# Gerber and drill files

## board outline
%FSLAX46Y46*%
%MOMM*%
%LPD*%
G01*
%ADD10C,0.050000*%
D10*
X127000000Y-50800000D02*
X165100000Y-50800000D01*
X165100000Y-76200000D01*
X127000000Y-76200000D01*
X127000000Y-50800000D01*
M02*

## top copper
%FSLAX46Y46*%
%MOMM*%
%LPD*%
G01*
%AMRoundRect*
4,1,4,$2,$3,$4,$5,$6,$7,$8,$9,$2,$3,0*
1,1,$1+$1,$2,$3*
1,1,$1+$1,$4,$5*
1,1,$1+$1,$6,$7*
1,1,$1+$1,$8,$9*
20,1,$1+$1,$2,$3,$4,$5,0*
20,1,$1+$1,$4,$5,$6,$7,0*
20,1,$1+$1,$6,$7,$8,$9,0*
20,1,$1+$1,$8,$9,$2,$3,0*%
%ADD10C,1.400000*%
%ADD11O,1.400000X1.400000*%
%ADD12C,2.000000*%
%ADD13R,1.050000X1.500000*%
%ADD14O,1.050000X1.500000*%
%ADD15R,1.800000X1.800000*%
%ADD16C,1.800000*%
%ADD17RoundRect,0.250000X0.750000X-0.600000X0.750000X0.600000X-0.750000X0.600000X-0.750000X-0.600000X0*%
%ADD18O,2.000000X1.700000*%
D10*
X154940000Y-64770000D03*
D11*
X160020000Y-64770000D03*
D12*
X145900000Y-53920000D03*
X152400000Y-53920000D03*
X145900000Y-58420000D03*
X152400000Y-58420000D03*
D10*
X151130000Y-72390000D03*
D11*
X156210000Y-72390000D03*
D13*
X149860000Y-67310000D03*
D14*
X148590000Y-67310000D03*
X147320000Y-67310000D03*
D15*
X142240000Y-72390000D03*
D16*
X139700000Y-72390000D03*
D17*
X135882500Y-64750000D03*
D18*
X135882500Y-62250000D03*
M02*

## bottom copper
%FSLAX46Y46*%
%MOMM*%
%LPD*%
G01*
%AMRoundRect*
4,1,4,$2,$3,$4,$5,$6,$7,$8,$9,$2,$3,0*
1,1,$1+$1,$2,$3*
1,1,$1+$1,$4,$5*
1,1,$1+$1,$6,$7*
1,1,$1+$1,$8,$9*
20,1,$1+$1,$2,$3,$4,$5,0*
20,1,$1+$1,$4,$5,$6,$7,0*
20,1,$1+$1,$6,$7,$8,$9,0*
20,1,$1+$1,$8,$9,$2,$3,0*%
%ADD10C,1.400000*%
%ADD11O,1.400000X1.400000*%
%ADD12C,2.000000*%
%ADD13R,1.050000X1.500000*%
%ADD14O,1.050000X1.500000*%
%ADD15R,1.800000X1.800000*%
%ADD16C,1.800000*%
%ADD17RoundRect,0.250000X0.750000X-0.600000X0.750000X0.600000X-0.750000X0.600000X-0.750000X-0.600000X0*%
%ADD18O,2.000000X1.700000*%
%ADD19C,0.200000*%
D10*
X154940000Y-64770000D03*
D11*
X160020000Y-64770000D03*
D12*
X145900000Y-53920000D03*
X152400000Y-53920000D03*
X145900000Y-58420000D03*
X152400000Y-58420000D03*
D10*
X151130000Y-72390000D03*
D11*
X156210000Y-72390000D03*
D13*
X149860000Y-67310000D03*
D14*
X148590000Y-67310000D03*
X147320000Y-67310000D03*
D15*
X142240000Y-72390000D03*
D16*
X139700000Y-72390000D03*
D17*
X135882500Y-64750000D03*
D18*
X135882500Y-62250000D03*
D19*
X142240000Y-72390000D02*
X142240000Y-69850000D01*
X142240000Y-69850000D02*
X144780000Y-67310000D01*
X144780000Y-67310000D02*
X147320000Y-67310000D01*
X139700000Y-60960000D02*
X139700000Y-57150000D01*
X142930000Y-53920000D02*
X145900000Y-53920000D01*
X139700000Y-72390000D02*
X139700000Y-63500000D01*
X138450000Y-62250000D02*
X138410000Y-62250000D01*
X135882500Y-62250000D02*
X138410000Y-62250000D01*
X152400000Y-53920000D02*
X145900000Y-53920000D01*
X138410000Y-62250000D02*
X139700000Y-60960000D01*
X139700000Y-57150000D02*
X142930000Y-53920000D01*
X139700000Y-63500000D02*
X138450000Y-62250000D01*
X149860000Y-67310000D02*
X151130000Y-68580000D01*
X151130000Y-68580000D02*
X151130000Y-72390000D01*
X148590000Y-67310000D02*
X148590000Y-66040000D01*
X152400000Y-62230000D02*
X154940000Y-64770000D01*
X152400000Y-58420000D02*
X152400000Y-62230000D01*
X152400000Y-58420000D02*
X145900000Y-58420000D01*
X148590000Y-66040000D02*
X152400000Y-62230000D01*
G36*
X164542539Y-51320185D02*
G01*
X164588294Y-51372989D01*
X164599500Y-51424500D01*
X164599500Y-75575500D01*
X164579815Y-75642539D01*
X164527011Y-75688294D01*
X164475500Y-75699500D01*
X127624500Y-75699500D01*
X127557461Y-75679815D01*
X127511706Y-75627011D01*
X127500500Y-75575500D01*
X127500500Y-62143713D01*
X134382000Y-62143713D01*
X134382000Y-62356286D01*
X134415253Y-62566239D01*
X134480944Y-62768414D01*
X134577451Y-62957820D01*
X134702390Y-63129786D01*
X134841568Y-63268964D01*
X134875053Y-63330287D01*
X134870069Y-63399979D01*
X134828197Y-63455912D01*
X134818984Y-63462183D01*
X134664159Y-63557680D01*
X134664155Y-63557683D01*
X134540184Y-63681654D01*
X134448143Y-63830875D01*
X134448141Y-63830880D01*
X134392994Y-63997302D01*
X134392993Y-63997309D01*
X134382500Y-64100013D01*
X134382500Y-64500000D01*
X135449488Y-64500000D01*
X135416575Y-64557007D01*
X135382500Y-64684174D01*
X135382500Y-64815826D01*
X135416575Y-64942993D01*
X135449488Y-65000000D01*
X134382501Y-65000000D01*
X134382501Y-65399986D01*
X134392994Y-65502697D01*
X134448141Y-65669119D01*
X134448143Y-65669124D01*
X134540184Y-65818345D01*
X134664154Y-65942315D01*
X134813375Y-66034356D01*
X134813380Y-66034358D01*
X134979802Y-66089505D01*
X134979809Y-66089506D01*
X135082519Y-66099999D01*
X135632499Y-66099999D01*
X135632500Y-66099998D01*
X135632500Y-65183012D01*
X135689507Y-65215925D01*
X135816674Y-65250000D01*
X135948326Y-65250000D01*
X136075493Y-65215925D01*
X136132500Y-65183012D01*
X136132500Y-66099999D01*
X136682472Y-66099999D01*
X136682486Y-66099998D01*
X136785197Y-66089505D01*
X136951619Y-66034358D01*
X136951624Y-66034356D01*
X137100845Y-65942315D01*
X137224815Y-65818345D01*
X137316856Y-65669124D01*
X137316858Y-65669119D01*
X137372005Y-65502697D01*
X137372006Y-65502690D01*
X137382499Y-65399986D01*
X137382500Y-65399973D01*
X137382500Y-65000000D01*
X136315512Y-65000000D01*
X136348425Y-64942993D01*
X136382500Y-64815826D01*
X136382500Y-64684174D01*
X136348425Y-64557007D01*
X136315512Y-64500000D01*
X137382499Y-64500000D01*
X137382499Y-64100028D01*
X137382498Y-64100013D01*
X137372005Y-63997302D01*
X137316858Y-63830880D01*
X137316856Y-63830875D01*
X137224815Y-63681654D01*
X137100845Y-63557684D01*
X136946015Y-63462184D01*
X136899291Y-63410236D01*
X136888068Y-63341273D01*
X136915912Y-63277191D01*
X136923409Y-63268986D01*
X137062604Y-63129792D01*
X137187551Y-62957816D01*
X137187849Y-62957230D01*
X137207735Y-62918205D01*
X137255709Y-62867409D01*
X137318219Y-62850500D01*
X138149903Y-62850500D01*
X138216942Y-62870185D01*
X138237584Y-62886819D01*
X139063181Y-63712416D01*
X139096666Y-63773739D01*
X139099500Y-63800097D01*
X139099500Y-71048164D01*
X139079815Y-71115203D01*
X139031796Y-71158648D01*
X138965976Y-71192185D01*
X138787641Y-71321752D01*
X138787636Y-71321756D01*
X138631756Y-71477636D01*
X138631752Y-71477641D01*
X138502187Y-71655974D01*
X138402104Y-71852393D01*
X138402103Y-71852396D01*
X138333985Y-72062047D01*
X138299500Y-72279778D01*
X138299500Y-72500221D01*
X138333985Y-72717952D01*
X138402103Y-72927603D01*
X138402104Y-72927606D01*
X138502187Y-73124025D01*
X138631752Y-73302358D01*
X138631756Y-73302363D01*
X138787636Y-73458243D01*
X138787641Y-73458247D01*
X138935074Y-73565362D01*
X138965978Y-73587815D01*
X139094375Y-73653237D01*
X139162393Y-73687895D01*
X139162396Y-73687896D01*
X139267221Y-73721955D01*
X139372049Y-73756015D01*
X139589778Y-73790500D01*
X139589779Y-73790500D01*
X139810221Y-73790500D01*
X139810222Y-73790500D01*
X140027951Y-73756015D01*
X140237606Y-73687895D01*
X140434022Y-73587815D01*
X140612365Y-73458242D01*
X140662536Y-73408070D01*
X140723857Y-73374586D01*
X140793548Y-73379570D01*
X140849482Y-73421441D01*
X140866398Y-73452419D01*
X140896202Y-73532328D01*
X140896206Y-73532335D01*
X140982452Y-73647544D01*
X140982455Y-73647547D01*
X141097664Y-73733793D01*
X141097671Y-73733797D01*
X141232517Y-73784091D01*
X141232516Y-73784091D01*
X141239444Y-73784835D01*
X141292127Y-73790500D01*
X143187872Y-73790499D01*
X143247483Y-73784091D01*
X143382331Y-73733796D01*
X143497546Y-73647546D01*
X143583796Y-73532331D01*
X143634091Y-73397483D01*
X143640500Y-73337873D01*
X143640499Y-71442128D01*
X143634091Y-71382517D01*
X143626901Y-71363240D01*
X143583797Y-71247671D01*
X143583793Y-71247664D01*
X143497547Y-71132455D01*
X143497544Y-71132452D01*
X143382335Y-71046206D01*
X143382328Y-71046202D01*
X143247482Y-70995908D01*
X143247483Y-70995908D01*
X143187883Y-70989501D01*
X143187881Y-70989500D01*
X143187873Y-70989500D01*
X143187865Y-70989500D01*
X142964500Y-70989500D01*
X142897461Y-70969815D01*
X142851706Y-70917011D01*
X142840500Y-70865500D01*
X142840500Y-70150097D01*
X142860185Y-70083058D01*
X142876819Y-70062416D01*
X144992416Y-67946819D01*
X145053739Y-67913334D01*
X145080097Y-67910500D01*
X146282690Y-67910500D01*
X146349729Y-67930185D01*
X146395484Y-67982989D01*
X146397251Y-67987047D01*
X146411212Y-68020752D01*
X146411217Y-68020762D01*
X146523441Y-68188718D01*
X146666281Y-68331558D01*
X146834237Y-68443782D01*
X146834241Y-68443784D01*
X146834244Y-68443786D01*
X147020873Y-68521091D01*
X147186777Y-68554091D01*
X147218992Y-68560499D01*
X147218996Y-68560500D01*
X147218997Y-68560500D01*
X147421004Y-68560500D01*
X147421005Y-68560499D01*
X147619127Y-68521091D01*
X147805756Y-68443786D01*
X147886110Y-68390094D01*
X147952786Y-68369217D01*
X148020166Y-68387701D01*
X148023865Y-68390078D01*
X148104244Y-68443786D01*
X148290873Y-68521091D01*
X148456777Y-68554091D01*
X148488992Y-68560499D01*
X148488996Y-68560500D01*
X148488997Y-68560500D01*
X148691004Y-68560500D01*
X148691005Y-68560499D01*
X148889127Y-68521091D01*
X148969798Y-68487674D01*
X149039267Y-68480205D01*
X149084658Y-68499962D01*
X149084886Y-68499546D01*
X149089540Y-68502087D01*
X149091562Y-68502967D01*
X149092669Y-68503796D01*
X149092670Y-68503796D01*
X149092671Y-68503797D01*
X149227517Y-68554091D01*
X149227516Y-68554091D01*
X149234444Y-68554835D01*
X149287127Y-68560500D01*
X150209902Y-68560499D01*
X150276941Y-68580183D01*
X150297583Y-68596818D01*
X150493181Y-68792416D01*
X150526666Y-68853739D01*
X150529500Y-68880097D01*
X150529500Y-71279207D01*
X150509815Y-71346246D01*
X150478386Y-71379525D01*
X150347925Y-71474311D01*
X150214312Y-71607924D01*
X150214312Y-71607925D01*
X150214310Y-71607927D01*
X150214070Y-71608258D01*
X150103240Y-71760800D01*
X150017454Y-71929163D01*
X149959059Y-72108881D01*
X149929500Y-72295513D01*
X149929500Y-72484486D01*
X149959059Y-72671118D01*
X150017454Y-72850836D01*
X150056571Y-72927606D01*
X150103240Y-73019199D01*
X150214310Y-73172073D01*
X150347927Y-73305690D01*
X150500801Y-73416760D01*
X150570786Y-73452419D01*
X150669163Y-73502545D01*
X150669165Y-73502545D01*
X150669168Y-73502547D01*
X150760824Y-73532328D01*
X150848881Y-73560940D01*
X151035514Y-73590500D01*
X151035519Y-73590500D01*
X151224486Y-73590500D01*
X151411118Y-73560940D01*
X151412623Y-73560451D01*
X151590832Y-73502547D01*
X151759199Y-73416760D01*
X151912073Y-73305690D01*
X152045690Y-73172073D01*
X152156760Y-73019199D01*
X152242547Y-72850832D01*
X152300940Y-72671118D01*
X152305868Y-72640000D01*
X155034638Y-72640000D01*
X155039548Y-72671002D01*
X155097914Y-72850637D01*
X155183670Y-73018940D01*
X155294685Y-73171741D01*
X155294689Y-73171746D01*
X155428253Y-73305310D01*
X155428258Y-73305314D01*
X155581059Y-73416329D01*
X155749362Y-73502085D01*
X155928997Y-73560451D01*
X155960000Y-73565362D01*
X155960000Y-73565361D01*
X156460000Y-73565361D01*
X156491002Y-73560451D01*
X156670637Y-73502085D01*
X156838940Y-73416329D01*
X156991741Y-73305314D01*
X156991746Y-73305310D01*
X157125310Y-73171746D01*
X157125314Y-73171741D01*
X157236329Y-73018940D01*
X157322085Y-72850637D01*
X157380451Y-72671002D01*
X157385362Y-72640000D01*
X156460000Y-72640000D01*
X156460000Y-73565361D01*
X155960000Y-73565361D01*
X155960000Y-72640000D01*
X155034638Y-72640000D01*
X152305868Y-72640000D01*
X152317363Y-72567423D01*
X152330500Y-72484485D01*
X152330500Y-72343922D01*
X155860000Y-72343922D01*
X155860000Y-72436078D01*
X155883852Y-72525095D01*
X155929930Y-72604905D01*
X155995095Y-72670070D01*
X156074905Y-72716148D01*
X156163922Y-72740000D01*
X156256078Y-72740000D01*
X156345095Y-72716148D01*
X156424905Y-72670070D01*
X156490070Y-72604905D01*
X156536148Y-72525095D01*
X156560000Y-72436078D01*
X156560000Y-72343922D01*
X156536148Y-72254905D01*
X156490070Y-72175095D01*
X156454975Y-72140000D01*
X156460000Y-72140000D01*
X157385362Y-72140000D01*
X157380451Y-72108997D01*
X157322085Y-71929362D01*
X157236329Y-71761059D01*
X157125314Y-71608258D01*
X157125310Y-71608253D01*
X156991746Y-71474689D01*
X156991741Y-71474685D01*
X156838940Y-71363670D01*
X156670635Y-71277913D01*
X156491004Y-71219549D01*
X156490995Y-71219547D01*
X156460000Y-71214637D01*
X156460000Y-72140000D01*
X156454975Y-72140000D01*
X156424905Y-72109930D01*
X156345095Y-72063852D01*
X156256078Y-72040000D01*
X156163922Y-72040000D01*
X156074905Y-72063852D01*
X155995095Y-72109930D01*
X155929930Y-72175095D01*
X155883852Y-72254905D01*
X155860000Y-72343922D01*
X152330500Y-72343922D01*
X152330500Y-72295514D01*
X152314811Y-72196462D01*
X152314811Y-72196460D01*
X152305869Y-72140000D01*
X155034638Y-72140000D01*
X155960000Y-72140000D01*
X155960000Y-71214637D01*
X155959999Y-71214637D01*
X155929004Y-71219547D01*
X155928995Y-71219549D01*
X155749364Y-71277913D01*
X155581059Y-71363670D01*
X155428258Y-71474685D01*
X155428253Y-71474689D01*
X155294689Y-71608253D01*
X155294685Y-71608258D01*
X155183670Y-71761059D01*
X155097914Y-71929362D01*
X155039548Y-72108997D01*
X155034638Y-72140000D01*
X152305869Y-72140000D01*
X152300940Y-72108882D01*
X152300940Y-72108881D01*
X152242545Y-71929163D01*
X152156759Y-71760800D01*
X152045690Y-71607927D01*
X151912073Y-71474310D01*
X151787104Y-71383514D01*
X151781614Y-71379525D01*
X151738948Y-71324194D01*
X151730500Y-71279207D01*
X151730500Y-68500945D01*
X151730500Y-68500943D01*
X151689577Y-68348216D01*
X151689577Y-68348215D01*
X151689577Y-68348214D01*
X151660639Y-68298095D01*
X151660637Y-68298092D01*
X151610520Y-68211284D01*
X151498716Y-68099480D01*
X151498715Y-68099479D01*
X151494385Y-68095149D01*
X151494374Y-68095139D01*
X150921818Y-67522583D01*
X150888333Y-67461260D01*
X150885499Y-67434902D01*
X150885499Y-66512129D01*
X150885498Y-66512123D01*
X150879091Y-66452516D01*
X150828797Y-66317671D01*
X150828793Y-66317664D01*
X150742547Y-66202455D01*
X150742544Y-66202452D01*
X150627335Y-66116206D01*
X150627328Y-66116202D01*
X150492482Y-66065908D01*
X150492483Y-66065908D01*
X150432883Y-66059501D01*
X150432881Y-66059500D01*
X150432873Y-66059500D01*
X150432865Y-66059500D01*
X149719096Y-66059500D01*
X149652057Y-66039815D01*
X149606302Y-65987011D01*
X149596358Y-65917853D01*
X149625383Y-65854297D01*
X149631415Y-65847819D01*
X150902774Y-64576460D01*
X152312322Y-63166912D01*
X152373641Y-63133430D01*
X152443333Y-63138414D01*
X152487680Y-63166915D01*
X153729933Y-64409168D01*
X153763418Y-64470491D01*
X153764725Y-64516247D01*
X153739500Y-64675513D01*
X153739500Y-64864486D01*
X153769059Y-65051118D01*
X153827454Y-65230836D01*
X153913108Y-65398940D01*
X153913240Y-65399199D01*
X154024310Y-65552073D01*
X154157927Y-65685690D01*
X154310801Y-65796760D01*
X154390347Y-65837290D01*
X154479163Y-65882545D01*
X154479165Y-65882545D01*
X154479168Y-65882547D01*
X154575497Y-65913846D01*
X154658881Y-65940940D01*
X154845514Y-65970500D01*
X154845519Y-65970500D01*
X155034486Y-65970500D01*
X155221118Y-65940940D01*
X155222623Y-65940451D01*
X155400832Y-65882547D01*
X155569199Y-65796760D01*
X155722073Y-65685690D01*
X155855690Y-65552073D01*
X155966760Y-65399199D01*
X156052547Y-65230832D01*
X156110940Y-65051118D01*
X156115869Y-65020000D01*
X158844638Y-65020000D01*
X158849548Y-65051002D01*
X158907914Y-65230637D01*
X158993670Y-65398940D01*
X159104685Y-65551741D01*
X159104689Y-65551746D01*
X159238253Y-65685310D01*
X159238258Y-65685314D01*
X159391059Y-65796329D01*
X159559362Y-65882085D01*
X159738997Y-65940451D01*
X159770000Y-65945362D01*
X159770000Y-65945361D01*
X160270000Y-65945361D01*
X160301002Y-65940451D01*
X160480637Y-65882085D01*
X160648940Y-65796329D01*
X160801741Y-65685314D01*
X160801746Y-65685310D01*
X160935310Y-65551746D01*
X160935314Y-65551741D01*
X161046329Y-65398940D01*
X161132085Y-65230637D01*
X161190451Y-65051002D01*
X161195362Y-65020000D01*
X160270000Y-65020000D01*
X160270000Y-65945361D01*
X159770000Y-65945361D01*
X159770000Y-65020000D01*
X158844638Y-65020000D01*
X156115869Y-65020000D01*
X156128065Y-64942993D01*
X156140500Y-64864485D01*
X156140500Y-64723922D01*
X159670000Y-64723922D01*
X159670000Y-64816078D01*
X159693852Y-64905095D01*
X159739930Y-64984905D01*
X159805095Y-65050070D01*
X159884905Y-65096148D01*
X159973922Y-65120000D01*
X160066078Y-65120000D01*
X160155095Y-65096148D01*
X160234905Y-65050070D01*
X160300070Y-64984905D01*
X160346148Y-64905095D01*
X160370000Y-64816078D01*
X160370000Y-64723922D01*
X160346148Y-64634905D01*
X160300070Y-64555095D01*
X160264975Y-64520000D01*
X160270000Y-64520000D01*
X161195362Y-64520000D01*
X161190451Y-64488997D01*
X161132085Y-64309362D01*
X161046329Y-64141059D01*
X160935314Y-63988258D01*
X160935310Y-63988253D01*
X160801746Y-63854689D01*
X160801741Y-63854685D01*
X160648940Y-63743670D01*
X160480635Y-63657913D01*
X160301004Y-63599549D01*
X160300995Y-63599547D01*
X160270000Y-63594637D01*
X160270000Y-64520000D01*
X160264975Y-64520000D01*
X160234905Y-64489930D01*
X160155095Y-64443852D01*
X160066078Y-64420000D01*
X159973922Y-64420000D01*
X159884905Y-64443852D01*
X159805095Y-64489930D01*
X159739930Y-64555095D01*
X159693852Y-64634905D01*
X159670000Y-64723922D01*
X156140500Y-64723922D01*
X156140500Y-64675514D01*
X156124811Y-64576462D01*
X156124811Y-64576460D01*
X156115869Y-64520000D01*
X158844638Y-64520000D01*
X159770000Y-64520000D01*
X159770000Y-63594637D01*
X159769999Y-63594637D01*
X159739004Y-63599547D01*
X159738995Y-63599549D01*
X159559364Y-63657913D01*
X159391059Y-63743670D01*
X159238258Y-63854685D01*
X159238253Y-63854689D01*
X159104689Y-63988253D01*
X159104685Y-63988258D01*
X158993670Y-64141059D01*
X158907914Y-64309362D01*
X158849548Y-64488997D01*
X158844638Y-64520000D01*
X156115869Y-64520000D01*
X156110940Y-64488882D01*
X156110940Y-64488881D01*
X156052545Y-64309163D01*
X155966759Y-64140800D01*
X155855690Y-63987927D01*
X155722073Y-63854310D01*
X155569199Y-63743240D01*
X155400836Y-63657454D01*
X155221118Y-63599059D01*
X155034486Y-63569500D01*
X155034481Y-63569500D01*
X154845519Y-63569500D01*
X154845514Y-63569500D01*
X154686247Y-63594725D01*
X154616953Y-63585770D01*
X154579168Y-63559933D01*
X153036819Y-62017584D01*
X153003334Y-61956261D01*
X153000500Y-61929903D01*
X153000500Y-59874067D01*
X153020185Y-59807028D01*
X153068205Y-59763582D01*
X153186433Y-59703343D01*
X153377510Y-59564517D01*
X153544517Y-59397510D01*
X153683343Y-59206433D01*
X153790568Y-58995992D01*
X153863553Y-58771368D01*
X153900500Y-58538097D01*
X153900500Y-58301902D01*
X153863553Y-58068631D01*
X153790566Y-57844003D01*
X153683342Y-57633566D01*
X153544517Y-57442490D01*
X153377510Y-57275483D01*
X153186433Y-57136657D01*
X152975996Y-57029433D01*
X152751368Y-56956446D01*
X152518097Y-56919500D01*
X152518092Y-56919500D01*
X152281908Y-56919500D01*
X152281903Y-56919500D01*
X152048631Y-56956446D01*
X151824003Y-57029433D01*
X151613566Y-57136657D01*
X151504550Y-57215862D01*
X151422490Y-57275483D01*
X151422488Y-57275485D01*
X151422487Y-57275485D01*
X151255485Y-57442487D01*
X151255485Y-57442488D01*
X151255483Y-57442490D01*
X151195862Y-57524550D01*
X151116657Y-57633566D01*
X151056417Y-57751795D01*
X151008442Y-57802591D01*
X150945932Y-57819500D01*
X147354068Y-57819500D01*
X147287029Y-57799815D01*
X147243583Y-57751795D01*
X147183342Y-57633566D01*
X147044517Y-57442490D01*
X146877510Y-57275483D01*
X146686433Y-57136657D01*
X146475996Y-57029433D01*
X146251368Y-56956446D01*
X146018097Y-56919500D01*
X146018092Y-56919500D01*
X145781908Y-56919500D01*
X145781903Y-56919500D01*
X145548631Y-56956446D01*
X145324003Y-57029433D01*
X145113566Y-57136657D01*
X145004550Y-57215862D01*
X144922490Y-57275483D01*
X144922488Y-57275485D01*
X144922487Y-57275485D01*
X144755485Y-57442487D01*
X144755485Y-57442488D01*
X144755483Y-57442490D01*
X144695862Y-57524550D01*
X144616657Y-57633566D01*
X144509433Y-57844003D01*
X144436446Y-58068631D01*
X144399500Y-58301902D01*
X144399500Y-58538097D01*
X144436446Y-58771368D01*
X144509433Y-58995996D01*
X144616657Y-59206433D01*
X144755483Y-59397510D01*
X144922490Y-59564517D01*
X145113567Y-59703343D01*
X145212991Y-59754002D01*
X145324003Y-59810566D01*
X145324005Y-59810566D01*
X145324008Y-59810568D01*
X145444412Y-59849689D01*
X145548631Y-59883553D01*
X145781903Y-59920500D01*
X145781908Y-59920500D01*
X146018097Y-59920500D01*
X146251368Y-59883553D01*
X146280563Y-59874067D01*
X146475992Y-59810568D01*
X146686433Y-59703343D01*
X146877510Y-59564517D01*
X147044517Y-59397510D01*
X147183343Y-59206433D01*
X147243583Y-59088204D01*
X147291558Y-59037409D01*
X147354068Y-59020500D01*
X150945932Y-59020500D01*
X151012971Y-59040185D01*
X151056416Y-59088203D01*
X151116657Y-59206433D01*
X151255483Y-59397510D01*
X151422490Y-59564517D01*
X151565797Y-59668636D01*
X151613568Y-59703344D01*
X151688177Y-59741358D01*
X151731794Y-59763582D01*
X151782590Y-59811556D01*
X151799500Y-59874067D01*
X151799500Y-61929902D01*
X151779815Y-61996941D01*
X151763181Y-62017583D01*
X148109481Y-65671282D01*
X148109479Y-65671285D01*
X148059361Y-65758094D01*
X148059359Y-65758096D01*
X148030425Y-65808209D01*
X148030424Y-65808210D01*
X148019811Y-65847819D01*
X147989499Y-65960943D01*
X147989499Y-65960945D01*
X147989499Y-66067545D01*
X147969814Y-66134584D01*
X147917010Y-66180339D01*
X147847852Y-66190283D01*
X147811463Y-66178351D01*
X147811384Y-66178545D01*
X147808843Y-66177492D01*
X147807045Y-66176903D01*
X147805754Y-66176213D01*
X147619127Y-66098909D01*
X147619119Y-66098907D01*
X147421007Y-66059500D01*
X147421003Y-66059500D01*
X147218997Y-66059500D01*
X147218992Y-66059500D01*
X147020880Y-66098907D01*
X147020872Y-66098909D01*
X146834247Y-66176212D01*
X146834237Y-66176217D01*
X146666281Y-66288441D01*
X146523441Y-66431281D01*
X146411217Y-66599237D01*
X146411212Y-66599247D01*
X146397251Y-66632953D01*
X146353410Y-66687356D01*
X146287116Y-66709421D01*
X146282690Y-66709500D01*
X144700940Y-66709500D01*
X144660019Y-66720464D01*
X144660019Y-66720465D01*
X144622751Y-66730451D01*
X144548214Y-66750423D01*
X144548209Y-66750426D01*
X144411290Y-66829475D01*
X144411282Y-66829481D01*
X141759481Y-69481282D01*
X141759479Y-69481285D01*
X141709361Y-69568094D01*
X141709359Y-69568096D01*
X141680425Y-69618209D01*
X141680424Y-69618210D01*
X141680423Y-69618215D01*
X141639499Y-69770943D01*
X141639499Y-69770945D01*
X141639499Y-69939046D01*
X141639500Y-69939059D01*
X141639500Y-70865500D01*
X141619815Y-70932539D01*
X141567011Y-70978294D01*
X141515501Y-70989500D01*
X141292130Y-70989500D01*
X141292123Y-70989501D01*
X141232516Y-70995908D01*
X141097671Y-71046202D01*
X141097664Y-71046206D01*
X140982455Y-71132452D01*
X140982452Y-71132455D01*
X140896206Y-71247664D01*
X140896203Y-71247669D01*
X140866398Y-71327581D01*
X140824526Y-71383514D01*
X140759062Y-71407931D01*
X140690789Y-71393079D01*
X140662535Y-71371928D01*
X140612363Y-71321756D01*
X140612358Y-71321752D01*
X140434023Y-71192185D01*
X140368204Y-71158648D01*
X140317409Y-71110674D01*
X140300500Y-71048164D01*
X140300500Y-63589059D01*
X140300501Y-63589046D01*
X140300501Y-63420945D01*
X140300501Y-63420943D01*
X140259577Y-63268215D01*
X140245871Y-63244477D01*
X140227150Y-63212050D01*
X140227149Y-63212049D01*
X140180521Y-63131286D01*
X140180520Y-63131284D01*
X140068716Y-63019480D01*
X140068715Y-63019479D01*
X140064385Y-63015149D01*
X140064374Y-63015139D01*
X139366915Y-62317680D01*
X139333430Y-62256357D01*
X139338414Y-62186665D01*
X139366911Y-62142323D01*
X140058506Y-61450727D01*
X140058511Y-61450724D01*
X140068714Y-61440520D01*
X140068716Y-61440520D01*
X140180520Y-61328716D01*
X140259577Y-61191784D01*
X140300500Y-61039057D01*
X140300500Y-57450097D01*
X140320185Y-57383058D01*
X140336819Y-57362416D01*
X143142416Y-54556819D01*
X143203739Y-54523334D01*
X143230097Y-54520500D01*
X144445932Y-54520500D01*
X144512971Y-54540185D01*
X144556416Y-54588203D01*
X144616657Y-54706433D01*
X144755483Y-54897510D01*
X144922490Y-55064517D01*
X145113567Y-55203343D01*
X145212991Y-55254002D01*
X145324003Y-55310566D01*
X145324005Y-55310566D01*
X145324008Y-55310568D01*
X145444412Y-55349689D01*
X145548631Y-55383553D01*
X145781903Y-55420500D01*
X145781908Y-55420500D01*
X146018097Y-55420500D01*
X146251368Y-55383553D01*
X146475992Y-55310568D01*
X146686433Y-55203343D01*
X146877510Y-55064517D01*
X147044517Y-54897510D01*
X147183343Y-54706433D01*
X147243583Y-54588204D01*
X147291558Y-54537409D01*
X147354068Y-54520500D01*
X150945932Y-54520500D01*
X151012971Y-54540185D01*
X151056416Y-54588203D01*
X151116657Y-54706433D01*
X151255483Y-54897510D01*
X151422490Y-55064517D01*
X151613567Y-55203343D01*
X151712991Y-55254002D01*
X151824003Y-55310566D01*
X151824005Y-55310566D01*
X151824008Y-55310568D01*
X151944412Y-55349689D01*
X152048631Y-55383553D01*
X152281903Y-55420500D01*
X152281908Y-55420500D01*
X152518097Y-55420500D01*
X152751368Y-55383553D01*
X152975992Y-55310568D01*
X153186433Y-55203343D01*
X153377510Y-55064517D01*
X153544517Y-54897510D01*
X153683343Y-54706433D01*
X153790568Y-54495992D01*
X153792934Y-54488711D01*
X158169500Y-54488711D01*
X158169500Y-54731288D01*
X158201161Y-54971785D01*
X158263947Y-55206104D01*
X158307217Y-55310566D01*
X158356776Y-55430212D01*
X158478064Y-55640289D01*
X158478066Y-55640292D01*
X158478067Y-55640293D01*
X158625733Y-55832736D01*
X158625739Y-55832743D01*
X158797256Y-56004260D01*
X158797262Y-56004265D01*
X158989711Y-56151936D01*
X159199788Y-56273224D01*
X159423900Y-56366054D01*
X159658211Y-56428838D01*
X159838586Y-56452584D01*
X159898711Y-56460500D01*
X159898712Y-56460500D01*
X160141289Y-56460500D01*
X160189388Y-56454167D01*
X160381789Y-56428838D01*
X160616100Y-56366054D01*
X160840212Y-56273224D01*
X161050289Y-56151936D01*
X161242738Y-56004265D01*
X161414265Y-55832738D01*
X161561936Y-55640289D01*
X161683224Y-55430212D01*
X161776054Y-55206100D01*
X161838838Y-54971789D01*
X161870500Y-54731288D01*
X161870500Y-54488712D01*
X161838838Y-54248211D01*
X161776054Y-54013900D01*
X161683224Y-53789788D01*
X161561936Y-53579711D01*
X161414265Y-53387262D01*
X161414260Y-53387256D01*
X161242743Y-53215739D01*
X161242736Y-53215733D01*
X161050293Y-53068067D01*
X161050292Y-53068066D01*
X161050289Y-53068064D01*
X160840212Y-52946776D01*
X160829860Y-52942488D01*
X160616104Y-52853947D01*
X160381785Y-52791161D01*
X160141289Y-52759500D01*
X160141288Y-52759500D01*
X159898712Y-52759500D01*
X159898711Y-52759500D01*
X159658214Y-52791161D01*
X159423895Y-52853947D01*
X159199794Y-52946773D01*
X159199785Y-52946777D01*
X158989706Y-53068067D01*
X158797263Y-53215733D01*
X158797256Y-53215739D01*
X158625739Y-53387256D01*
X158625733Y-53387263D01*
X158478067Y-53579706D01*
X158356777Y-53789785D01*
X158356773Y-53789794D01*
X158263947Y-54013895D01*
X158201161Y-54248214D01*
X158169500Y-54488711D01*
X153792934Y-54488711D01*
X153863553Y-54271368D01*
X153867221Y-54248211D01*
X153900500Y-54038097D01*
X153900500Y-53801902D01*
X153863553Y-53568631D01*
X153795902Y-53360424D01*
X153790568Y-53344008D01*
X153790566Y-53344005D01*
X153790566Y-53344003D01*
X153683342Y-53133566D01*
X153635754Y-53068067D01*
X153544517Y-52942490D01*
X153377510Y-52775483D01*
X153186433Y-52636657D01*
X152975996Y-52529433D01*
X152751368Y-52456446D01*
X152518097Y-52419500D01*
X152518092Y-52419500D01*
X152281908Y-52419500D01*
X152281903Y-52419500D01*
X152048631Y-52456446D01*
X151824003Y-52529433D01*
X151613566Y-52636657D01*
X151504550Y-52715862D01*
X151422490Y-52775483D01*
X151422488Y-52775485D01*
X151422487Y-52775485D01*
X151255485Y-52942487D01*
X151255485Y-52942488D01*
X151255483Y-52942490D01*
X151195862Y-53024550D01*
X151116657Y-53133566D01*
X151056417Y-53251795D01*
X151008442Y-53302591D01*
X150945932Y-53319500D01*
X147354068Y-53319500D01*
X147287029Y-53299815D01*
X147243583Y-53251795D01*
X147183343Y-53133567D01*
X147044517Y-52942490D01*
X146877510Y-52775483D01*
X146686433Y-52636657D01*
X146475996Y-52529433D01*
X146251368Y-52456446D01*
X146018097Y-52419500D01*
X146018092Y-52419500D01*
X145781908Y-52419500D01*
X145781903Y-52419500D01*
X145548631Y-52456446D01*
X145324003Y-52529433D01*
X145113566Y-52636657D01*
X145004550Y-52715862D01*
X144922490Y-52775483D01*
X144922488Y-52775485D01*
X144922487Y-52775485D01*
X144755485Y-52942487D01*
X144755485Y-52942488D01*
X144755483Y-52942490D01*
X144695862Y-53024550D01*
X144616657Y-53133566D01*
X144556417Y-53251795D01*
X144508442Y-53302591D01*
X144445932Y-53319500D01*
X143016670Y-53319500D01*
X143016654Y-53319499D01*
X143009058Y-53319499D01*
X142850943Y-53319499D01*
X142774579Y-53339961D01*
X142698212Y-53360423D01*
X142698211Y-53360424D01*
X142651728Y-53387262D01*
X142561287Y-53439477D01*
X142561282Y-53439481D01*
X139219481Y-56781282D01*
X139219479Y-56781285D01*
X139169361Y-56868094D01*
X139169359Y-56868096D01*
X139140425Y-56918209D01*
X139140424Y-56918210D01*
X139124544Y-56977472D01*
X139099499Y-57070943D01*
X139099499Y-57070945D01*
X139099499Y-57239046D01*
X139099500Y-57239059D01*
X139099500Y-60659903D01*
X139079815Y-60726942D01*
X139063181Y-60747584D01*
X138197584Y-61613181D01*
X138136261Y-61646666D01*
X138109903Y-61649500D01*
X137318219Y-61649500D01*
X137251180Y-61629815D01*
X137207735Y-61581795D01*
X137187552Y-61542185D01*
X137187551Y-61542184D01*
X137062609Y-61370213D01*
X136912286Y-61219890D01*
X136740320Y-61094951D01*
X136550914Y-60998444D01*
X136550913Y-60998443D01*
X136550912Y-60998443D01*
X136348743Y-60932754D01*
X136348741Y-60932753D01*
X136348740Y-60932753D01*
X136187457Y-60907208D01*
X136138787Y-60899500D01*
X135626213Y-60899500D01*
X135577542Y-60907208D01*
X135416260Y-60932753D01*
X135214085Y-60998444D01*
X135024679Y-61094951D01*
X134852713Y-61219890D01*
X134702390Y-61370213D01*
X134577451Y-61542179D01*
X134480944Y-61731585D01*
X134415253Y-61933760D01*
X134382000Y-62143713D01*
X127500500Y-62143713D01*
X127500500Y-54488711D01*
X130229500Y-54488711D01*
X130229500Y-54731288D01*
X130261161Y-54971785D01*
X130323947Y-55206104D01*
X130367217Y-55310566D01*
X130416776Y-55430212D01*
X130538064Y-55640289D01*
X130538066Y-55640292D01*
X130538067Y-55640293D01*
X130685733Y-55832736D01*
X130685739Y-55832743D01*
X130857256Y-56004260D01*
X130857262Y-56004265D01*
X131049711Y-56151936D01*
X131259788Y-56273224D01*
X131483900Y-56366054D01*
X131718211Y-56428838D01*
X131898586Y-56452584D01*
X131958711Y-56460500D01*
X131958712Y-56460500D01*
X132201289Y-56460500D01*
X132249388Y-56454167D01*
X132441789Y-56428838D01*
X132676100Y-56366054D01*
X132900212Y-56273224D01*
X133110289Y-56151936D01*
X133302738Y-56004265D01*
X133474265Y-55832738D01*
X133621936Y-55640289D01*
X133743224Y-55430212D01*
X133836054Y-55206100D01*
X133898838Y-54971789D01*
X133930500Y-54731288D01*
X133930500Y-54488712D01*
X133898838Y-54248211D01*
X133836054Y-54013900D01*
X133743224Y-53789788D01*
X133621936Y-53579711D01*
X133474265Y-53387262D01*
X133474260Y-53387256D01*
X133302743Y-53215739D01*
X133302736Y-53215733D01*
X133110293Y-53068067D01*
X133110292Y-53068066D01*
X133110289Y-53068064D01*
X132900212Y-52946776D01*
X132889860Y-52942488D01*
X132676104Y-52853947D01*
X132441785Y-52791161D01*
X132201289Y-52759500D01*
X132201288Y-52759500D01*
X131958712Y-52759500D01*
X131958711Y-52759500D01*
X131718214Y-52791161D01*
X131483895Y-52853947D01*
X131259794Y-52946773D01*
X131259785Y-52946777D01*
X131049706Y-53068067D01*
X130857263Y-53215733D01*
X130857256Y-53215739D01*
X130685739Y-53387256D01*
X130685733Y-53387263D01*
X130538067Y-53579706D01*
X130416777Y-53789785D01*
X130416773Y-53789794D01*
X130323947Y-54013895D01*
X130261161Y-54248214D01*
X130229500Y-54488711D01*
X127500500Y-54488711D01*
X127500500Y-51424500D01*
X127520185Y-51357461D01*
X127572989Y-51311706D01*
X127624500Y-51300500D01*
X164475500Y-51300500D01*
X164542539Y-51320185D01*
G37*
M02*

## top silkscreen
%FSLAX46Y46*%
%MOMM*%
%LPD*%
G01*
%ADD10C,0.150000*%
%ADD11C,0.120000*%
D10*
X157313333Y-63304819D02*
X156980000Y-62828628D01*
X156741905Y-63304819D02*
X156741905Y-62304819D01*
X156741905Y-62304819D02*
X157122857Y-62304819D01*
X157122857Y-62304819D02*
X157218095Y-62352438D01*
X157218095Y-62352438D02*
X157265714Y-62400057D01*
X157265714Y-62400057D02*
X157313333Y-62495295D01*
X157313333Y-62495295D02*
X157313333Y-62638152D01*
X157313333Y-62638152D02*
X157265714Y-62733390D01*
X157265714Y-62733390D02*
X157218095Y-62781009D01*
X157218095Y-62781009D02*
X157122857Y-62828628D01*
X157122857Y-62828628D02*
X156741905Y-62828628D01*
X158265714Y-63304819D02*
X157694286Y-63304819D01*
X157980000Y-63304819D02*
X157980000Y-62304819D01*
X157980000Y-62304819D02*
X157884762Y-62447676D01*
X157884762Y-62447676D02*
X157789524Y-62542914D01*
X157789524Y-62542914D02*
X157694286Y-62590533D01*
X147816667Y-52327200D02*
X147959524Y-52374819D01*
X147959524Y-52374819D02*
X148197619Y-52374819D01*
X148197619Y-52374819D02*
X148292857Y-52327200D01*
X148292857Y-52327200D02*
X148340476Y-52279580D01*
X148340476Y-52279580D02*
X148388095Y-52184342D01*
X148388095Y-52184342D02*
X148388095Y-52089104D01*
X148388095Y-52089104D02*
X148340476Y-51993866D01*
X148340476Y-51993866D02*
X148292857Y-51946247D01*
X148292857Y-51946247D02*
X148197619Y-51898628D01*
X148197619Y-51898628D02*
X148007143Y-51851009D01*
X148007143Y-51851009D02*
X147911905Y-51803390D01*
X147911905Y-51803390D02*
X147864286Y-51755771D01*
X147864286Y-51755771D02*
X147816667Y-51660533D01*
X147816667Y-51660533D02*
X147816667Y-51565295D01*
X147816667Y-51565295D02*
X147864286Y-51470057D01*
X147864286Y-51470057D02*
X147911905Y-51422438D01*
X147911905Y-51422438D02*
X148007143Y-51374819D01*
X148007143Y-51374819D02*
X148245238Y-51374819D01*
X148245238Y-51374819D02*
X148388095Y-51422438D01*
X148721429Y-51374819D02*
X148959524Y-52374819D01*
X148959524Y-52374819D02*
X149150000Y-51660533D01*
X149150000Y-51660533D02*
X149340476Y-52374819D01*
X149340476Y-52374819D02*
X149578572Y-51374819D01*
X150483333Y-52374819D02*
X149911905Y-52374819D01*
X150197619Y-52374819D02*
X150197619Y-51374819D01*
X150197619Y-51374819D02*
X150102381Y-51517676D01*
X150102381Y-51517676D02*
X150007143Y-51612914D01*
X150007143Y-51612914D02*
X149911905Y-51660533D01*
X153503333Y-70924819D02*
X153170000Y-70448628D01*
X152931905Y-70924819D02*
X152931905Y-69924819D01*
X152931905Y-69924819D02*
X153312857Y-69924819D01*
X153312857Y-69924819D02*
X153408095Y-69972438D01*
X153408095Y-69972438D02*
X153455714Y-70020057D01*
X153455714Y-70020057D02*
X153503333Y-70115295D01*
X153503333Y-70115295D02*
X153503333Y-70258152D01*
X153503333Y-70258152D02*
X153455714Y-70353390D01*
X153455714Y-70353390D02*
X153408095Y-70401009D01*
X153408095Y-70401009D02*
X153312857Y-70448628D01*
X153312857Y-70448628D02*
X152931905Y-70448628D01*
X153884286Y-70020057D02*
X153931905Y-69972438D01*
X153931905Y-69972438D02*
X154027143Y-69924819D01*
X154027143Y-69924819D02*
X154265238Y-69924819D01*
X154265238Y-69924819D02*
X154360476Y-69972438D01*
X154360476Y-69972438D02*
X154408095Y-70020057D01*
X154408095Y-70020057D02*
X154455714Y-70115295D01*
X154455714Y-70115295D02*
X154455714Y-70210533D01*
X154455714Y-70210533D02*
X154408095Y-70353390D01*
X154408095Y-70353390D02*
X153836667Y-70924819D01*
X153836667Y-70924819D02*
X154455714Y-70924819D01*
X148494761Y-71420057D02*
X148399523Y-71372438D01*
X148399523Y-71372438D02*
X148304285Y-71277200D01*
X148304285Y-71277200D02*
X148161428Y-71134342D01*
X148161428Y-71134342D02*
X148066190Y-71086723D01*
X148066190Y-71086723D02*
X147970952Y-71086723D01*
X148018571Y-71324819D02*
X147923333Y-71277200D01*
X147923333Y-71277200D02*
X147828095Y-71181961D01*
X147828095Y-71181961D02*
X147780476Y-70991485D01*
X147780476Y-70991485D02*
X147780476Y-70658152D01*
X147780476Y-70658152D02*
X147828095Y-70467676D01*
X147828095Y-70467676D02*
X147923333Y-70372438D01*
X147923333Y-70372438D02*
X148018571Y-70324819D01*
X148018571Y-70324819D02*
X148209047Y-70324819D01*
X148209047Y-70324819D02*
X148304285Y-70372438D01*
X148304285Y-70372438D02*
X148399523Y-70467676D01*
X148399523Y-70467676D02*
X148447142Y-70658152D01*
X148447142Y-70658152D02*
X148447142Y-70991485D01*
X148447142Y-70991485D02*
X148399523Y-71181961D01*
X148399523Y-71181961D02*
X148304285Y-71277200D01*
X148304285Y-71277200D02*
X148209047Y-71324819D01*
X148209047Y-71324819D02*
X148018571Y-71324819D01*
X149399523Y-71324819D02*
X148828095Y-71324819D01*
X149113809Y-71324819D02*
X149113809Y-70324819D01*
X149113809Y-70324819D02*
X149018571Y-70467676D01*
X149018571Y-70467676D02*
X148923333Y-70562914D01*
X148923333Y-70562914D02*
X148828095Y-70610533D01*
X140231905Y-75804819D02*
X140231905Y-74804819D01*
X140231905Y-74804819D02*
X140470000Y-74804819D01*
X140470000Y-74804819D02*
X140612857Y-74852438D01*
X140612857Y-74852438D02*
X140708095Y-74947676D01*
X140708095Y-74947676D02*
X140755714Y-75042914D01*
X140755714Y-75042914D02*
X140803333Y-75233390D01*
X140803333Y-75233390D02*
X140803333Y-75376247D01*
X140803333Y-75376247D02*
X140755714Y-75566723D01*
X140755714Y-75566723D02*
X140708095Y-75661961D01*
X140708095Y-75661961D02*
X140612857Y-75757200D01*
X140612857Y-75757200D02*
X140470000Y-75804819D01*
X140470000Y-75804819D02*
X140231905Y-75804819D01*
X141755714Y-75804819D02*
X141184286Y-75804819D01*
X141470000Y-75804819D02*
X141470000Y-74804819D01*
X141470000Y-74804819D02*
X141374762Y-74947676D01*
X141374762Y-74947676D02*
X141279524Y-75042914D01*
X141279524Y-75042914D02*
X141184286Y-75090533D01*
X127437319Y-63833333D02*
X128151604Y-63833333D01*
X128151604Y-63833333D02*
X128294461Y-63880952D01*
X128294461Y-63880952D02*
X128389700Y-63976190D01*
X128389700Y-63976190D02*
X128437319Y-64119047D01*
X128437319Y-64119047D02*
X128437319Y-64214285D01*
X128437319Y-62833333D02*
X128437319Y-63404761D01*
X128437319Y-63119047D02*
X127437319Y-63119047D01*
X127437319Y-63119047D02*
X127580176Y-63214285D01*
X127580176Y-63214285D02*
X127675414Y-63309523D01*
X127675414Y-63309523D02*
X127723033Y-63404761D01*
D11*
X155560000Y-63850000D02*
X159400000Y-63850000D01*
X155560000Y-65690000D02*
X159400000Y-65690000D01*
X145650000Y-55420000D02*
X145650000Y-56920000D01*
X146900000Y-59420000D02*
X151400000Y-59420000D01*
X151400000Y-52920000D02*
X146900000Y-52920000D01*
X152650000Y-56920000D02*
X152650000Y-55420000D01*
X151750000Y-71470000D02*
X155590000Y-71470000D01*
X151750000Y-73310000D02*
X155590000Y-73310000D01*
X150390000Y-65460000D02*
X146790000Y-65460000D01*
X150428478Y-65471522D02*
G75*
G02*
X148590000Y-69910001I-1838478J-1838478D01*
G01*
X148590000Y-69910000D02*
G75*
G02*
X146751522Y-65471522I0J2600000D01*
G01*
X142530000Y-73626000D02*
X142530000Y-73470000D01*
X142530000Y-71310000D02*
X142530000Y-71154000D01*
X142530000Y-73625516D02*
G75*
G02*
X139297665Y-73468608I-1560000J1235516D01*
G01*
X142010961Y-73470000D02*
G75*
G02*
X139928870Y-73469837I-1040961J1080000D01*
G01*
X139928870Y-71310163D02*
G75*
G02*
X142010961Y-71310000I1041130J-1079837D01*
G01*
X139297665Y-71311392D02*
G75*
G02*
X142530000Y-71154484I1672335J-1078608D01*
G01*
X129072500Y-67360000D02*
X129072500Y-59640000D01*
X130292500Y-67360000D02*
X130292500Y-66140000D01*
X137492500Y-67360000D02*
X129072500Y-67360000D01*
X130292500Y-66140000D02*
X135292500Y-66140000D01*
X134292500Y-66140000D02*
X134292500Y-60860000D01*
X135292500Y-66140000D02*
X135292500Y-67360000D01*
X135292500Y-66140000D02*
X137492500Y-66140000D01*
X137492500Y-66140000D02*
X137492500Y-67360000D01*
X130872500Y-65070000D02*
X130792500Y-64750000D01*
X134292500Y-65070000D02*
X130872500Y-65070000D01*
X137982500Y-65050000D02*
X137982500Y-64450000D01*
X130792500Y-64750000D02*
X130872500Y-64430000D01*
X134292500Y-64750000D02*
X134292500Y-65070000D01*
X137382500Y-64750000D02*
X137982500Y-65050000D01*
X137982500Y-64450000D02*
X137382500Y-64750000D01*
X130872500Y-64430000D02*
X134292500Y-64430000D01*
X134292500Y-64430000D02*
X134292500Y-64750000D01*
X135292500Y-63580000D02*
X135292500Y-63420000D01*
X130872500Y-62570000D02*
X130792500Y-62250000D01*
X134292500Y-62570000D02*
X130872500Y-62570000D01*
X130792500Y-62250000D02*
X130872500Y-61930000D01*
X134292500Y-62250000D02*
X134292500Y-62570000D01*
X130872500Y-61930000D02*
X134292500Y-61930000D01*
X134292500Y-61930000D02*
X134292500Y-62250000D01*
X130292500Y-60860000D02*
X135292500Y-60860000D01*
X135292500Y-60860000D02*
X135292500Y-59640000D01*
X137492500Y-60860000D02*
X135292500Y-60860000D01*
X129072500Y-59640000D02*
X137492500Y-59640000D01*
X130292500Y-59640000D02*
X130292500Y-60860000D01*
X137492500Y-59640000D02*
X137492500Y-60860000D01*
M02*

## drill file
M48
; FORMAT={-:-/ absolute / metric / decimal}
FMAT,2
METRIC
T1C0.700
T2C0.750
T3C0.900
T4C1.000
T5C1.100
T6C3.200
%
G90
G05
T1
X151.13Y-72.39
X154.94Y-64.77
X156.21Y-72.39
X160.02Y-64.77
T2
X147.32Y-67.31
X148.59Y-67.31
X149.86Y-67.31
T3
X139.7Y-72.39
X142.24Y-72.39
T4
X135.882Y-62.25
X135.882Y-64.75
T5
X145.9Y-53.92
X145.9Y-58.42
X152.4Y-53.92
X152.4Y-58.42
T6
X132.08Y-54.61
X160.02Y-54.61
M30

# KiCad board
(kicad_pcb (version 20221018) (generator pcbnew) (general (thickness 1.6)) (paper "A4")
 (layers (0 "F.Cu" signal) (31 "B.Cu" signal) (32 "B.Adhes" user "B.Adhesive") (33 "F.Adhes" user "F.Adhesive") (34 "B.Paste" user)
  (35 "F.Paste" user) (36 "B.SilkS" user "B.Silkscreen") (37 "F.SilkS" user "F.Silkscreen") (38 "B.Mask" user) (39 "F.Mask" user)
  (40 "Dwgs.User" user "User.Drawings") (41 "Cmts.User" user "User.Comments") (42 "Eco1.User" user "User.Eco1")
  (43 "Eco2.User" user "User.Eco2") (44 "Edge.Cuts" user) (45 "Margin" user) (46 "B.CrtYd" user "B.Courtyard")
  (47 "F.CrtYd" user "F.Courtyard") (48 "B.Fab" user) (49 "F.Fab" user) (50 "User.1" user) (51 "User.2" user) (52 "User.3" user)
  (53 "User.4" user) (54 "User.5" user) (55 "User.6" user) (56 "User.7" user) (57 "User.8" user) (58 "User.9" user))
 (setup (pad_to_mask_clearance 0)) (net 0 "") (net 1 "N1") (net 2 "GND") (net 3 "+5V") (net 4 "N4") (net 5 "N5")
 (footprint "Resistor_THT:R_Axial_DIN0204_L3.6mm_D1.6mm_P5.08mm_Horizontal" (layer "F.Cu") (at 154.94 64.77)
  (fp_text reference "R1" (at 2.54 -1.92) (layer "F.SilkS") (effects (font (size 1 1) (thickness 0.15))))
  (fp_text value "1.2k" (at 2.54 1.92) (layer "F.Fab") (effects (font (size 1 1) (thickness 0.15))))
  (fp_line (start 0.62 -0.92) (end 4.46 -0.92) (stroke (width 0.12) (type solid)) (layer "F.SilkS"))
  (fp_line (start 0.62 0.92) (end 4.46 0.92) (stroke (width 0.12) (type solid)) (layer "F.SilkS"))
  (pad "1" thru_hole circle (at 0 0) (size 1.4 1.4) (drill 0.7) (layers "*.Cu" "*.Mask") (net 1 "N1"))
  (pad "2" thru_hole oval (at 5.08 0) (size 1.4 1.4) (drill 0.7) (layers "*.Cu" "*.Mask") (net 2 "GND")))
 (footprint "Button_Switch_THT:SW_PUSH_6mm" (layer "F.Cu") (at 145.9 53.92)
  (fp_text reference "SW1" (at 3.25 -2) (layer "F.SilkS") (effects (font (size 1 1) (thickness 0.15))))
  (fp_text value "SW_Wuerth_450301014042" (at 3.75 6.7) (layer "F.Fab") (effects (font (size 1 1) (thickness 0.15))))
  (fp_line (start -0.25 1.5) (end -0.25 3) (stroke (width 0.12) (type solid)) (layer "F.SilkS"))
  (fp_line (start 1 5.5) (end 5.5 5.5) (stroke (width 0.12) (type solid)) (layer "F.SilkS"))
  (fp_line (start 5.5 -1) (end 1 -1) (stroke (width 0.12) (type solid)) (layer "F.SilkS"))
  (fp_line (start 6.75 3) (end 6.75 1.5) (stroke (width 0.12) (type solid)) (layer "F.SilkS"))
  (pad "1" thru_hole circle (at 0 0 90) (size 2 2) (drill 1.1) (layers "*.Cu" "*.Mask") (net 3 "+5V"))
  (pad "1" thru_hole circle (at 6.5 0 90) (size 2 2) (drill 1.1) (layers "*.Cu" "*.Mask") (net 3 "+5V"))
  (pad "2" thru_hole circle (at 0 4.5 90) (size 2 2) (drill 1.1) (layers "*.Cu" "*.Mask") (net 1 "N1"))
  (pad "2" thru_hole circle (at 6.5 4.5 90) (size 2 2) (drill 1.1) (layers "*.Cu" "*.Mask") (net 1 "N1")))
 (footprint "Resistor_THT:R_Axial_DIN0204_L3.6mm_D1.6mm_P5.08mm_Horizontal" (layer "F.Cu") (at 151.13 72.39)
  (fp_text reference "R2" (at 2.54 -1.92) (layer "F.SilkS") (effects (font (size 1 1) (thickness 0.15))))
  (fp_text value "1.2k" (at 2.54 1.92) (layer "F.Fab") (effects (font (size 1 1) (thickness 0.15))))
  (fp_line (start 0.62 -0.92) (end 4.46 -0.92) (stroke (width 0.12) (type solid)) (layer "F.SilkS"))
  (fp_line (start 0.62 0.92) (end 4.46 0.92) (stroke (width 0.12) (type solid)) (layer "F.SilkS"))
  (pad "1" thru_hole circle (at 0 0) (size 1.4 1.4) (drill 0.7) (layers "*.Cu" "*.Mask") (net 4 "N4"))
  (pad "2" thru_hole oval (at 5.08 0) (size 1.4 1.4) (drill 0.7) (layers "*.Cu" "*.Mask") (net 2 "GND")))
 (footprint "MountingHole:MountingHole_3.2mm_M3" (layer "F.Cu") (at 160.02 54.61)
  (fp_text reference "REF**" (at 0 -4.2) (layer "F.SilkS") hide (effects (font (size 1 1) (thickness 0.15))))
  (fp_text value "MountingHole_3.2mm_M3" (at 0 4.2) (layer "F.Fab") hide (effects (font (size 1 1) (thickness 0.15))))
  (pad "" np_thru_hole circle (at 0 0) (size 3.2 3.2) (drill 3.2) (layers "*.Cu" "*.Mask")))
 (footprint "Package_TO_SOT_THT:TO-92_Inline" (layer "F.Cu") (at 149.86 67.31 180)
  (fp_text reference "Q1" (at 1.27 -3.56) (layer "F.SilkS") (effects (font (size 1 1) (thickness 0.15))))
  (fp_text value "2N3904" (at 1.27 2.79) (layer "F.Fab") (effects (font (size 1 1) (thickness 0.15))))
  (fp_line (start -0.53 1.85) (end 3.07 1.85) (stroke (width 0.12) (type solid)) (layer "F.SilkS"))
  (fp_arc (start -0.568478 1.838478) (mid -1.132087 -0.994977) (end 1.27 -2.6) (stroke (width 0.12) (type solid)) (layer "F.SilkS"))
  (fp_arc (start 1.27 -2.6) (mid 3.672087 -0.994977) (end 3.108478 1.838478) (stroke (width 0.12) (type solid)) (layer "F.SilkS"))
  (pad "1" thru_hole rect (at 0 0 180) (size 1.05 1.5) (drill 0.75) (layers "*.Cu" "*.Mask") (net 4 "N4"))
  (pad "2" thru_hole oval (at 1.27 0 180) (size 1.05 1.5) (drill 0.75) (layers "*.Cu" "*.Mask") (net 1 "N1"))
  (pad "3" thru_hole oval (at 2.54 0 180) (size 1.05 1.5) (drill 0.75) (layers "*.Cu" "*.Mask") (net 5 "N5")))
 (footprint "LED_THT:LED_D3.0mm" (layer "F.Cu") (at 142.24 72.39 180)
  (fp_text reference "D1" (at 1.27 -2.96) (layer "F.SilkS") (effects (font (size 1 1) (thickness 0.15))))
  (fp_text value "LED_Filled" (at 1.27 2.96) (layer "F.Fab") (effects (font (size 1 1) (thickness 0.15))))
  (fp_line (start -0.29 -1.236) (end -0.29 -1.08) (stroke (width 0.12) (type solid)) (layer "F.SilkS"))
  (fp_line (start -0.29 1.08) (end -0.29 1.236) (stroke (width 0.12) (type solid)) (layer "F.SilkS"))
  (fp_arc (start -0.29 -1.235516) (mid 1.366487 -1.987659) (end 2.942335 -1.078608) (stroke (width 0.12) (type solid)) (layer "F.SilkS"))
  (fp_arc (start 0.229039 -1.08) (mid 1.270117 -1.5) (end 2.31113 -1.079837) (stroke (width 0.12) (type solid)) (layer "F.SilkS"))
  (fp_arc (start 2.31113 1.079837) (mid 1.270117 1.5) (end 0.229039 1.08) (stroke (width 0.12) (type solid)) (layer "F.SilkS"))
  (fp_arc (start 2.942335 1.078608) (mid 1.366487 1.987659) (end -0.29 1.235516) (stroke (width 0.12) (type solid)) (layer "F.SilkS"))
  (pad "1" thru_hole rect (at 0 0 180) (size 1.8 1.8) (drill 0.9) (layers "*.Cu" "*.Mask") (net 5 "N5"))
  (pad "2" thru_hole circle (at 2.54 0 180) (size 1.8 1.8) (drill 0.9) (layers "*.Cu" "*.Mask") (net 3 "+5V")))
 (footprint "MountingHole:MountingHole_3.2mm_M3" (layer "F.Cu") (at 132.08 54.61)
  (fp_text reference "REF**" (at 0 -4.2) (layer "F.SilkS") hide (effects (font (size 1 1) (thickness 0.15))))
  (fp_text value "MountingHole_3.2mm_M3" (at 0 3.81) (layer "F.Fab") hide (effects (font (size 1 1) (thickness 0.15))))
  (pad "" np_thru_hole circle (at 0 0) (size 3.2 3.2) (drill 3.2) (layers "*.Cu" "*.Mask")))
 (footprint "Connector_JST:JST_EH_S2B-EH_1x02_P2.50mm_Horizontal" (layer "F.Cu") (at 135.8825 64.75 90)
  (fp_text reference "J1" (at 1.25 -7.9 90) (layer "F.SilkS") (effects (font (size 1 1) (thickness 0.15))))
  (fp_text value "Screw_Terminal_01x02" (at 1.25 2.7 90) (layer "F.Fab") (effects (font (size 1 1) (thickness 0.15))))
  (fp_line (start -2.61 -6.81) (end 5.11 -6.81) (stroke (width 0.12) (type solid)) (layer "F.SilkS"))
  (fp_line (start -2.61 -5.59) (end -1.39 -5.59) (stroke (width 0.12) (type solid)) (layer "F.SilkS"))
  (fp_line (start -2.61 1.61) (end -2.61 -6.81) (stroke (width 0.12) (type solid)) (layer "F.SilkS"))
  (fp_line (start -1.39 -5.59) (end -1.39 -0.59) (stroke (width 0.12) (type solid)) (layer "F.SilkS"))
  (fp_line (start -1.39 -1.59) (end 3.89 -1.59) (stroke (width 0.12) (type solid)) (layer "F.SilkS"))
  (fp_line (start -1.39 -0.59) (end -2.61 -0.59) (stroke (width 0.12) (type solid)) (layer "F.SilkS"))
  (fp_line (start -1.39 -0.59) (end -1.39 1.61) (stroke (width 0.12) (type solid)) (layer "F.SilkS"))
  (fp_line (start -1.39 1.61) (end -2.61 1.61) (stroke (width 0.12) (type solid)) (layer "F.SilkS"))
  (fp_line (start -0.32 -5.01) (end 0 -5.09) (stroke (width 0.12) (type solid)) (layer "F.SilkS"))
  (fp_line (start -0.32 -1.59) (end -0.32 -5.01) (stroke (width 0.12) (type solid)) (layer "F.SilkS"))
  (fp_line (start -0.3 2.1) (end 0.3 2.1) (stroke (width 0.12) (type solid)) (layer "F.SilkS"))
  (fp_line (start 0 -5.09) (end 0.32 -5.01) (stroke (width 0.12) (type solid)) (layer "F.SilkS"))
  (fp_line (start 0 -1.59) (end -0.32 -1.59) (stroke (width 0.12) (type solid)) (layer "F.SilkS"))
  (fp_line (start 0 1.5) (end -0.3 2.1) (stroke (width 0.12) (type solid)) (layer "F.SilkS"))
  (fp_line (start 0.3 2.1) (end 0 1.5) (stroke (width 0.12) (type solid)) (layer "F.SilkS"))
  (fp_line (start 0.32 -5.01) (end 0.32 -1.59) (stroke (width 0.12) (type solid)) (layer "F.SilkS"))
  (fp_line (start 0.32 -1.59) (end 0 -1.59) (stroke (width 0.12) (type solid)) (layer "F.SilkS"))
  (fp_line (start 1.17 -0.59) (end 1.33 -0.59) (stroke (width 0.12) (type solid)) (layer "F.SilkS"))
  (fp_line (start 2.18 -5.01) (end 2.5 -5.09) (stroke (width 0.12) (type solid)) (layer "F.SilkS"))
  (fp_line (start 2.18 -1.59) (end 2.18 -5.01) (stroke (width 0.12) (type solid)) (layer "F.SilkS"))
  (fp_line (start 2.5 -5.09) (end 2.82 -5.01) (stroke (width 0.12) (type solid)) (layer "F.SilkS"))
  (fp_line (start 2.5 -1.59) (end 2.18 -1.59) (stroke (width 0.12) (type solid)) (layer "F.SilkS"))
  (fp_line (start 2.82 -5.01) (end 2.82 -1.59) (stroke (width 0.12) (type solid)) (layer "F.SilkS"))
  (fp_line (start 2.82 -1.59) (end 2.5 -1.59) (stroke (width 0.12) (type solid)) (layer "F.SilkS"))
  (fp_line (start 3.89 -5.59) (end 3.89 -0.59) (stroke (width 0.12) (type solid)) (layer "F.SilkS"))
  (fp_line (start 3.89 -0.59) (end 5.11 -0.59) (stroke (width 0.12) (type solid)) (layer "F.SilkS"))
  (fp_line (start 3.89 1.61) (end 3.89 -0.59) (stroke (width 0.12) (type solid)) (layer "F.SilkS"))
  (fp_line (start 5.11 -6.81) (end 5.11 1.61) (stroke (width 0.12) (type solid)) (layer "F.SilkS"))
  (fp_line (start 5.11 -5.59) (end 3.89 -5.59) (stroke (width 0.12) (type solid)) (layer "F.SilkS"))
  (fp_line (start 5.11 1.61) (end 3.89 1.61) (stroke (width 0.12) (type solid)) (layer "F.SilkS"))
  (pad "1" thru_hole roundrect (at 0 0 90) (size 1.7 2) (drill 1) (layers "*.Cu" "*.Mask") (roundrect_rratio 0.147059) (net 2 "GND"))
  (pad "2" thru_hole oval (at 2.5 0 90) (size 1.7 2) (drill 1) (layers "*.Cu" "*.Mask") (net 3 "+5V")))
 (gr_rect (start 127 50.8) (end 165.1 76.2) (stroke (width 0.05) (type default)) (fill none) (layer "Edge.Cuts"))
 (segment (start 142.24 72.39) (end 142.24 69.85) (width 0.2) (layer "B.Cu") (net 5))
 (segment (start 142.24 69.85) (end 144.78 67.31) (width 0.2) (layer "B.Cu") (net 5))
 (segment (start 144.78 67.31) (end 147.32 67.31) (width 0.2) (layer "B.Cu") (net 5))
 (segment (start 139.7 60.96) (end 139.7 57.15) (width 0.2) (layer "B.Cu") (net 3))
 (segment (start 142.93 53.92) (end 145.9 53.92) (width 0.2) (layer "B.Cu") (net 3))
 (segment (start 139.7 72.39) (end 139.7 63.5) (width 0.2) (layer "B.Cu") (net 3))
 (segment (start 138.45 62.25) (end 138.41 62.25) (width 0.2) (layer "B.Cu") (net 3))
 (segment (start 135.8825 62.25) (end 138.41 62.25) (width 0.2) (layer "B.Cu") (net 3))
 (segment (start 152.4 53.92) (end 145.9 53.92) (width 0.2) (layer "B.Cu") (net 3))
 (segment (start 138.41 62.25) (end 139.7 60.96) (width 0.2) (layer "B.Cu") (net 3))
 (segment (start 139.7 57.15) (end 142.93 53.92) (width 0.2) (layer "B.Cu") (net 3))
 (segment (start 139.7 63.5) (end 138.45 62.25) (width 0.2) (layer "B.Cu") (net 3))
 (segment (start 149.86 67.31) (end 151.13 68.58) (width 0.2) (layer "B.Cu") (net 4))
 (segment (start 151.13 68.58) (end 151.13 72.39) (width 0.2) (layer "B.Cu") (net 4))
 (segment (start 148.59 67.31) (end 148.59 66.04) (width 0.2) (layer "B.Cu") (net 1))
 (segment (start 152.4 62.23) (end 154.94 64.77) (width 0.2) (layer "B.Cu") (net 1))
 (segment (start 152.4 58.42) (end 152.4 62.23) (width 0.2) (layer "B.Cu") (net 1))
 (segment (start 152.4 58.42) (end 145.9 58.42) (width 0.2) (layer "B.Cu") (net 1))
 (segment (start 148.59 66.04) (end 152.4 62.23) (width 0.2) (layer "B.Cu") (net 1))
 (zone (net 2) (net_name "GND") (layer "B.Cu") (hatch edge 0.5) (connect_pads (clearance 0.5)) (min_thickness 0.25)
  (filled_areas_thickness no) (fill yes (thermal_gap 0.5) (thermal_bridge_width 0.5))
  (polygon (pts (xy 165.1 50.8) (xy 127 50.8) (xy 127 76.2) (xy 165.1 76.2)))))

